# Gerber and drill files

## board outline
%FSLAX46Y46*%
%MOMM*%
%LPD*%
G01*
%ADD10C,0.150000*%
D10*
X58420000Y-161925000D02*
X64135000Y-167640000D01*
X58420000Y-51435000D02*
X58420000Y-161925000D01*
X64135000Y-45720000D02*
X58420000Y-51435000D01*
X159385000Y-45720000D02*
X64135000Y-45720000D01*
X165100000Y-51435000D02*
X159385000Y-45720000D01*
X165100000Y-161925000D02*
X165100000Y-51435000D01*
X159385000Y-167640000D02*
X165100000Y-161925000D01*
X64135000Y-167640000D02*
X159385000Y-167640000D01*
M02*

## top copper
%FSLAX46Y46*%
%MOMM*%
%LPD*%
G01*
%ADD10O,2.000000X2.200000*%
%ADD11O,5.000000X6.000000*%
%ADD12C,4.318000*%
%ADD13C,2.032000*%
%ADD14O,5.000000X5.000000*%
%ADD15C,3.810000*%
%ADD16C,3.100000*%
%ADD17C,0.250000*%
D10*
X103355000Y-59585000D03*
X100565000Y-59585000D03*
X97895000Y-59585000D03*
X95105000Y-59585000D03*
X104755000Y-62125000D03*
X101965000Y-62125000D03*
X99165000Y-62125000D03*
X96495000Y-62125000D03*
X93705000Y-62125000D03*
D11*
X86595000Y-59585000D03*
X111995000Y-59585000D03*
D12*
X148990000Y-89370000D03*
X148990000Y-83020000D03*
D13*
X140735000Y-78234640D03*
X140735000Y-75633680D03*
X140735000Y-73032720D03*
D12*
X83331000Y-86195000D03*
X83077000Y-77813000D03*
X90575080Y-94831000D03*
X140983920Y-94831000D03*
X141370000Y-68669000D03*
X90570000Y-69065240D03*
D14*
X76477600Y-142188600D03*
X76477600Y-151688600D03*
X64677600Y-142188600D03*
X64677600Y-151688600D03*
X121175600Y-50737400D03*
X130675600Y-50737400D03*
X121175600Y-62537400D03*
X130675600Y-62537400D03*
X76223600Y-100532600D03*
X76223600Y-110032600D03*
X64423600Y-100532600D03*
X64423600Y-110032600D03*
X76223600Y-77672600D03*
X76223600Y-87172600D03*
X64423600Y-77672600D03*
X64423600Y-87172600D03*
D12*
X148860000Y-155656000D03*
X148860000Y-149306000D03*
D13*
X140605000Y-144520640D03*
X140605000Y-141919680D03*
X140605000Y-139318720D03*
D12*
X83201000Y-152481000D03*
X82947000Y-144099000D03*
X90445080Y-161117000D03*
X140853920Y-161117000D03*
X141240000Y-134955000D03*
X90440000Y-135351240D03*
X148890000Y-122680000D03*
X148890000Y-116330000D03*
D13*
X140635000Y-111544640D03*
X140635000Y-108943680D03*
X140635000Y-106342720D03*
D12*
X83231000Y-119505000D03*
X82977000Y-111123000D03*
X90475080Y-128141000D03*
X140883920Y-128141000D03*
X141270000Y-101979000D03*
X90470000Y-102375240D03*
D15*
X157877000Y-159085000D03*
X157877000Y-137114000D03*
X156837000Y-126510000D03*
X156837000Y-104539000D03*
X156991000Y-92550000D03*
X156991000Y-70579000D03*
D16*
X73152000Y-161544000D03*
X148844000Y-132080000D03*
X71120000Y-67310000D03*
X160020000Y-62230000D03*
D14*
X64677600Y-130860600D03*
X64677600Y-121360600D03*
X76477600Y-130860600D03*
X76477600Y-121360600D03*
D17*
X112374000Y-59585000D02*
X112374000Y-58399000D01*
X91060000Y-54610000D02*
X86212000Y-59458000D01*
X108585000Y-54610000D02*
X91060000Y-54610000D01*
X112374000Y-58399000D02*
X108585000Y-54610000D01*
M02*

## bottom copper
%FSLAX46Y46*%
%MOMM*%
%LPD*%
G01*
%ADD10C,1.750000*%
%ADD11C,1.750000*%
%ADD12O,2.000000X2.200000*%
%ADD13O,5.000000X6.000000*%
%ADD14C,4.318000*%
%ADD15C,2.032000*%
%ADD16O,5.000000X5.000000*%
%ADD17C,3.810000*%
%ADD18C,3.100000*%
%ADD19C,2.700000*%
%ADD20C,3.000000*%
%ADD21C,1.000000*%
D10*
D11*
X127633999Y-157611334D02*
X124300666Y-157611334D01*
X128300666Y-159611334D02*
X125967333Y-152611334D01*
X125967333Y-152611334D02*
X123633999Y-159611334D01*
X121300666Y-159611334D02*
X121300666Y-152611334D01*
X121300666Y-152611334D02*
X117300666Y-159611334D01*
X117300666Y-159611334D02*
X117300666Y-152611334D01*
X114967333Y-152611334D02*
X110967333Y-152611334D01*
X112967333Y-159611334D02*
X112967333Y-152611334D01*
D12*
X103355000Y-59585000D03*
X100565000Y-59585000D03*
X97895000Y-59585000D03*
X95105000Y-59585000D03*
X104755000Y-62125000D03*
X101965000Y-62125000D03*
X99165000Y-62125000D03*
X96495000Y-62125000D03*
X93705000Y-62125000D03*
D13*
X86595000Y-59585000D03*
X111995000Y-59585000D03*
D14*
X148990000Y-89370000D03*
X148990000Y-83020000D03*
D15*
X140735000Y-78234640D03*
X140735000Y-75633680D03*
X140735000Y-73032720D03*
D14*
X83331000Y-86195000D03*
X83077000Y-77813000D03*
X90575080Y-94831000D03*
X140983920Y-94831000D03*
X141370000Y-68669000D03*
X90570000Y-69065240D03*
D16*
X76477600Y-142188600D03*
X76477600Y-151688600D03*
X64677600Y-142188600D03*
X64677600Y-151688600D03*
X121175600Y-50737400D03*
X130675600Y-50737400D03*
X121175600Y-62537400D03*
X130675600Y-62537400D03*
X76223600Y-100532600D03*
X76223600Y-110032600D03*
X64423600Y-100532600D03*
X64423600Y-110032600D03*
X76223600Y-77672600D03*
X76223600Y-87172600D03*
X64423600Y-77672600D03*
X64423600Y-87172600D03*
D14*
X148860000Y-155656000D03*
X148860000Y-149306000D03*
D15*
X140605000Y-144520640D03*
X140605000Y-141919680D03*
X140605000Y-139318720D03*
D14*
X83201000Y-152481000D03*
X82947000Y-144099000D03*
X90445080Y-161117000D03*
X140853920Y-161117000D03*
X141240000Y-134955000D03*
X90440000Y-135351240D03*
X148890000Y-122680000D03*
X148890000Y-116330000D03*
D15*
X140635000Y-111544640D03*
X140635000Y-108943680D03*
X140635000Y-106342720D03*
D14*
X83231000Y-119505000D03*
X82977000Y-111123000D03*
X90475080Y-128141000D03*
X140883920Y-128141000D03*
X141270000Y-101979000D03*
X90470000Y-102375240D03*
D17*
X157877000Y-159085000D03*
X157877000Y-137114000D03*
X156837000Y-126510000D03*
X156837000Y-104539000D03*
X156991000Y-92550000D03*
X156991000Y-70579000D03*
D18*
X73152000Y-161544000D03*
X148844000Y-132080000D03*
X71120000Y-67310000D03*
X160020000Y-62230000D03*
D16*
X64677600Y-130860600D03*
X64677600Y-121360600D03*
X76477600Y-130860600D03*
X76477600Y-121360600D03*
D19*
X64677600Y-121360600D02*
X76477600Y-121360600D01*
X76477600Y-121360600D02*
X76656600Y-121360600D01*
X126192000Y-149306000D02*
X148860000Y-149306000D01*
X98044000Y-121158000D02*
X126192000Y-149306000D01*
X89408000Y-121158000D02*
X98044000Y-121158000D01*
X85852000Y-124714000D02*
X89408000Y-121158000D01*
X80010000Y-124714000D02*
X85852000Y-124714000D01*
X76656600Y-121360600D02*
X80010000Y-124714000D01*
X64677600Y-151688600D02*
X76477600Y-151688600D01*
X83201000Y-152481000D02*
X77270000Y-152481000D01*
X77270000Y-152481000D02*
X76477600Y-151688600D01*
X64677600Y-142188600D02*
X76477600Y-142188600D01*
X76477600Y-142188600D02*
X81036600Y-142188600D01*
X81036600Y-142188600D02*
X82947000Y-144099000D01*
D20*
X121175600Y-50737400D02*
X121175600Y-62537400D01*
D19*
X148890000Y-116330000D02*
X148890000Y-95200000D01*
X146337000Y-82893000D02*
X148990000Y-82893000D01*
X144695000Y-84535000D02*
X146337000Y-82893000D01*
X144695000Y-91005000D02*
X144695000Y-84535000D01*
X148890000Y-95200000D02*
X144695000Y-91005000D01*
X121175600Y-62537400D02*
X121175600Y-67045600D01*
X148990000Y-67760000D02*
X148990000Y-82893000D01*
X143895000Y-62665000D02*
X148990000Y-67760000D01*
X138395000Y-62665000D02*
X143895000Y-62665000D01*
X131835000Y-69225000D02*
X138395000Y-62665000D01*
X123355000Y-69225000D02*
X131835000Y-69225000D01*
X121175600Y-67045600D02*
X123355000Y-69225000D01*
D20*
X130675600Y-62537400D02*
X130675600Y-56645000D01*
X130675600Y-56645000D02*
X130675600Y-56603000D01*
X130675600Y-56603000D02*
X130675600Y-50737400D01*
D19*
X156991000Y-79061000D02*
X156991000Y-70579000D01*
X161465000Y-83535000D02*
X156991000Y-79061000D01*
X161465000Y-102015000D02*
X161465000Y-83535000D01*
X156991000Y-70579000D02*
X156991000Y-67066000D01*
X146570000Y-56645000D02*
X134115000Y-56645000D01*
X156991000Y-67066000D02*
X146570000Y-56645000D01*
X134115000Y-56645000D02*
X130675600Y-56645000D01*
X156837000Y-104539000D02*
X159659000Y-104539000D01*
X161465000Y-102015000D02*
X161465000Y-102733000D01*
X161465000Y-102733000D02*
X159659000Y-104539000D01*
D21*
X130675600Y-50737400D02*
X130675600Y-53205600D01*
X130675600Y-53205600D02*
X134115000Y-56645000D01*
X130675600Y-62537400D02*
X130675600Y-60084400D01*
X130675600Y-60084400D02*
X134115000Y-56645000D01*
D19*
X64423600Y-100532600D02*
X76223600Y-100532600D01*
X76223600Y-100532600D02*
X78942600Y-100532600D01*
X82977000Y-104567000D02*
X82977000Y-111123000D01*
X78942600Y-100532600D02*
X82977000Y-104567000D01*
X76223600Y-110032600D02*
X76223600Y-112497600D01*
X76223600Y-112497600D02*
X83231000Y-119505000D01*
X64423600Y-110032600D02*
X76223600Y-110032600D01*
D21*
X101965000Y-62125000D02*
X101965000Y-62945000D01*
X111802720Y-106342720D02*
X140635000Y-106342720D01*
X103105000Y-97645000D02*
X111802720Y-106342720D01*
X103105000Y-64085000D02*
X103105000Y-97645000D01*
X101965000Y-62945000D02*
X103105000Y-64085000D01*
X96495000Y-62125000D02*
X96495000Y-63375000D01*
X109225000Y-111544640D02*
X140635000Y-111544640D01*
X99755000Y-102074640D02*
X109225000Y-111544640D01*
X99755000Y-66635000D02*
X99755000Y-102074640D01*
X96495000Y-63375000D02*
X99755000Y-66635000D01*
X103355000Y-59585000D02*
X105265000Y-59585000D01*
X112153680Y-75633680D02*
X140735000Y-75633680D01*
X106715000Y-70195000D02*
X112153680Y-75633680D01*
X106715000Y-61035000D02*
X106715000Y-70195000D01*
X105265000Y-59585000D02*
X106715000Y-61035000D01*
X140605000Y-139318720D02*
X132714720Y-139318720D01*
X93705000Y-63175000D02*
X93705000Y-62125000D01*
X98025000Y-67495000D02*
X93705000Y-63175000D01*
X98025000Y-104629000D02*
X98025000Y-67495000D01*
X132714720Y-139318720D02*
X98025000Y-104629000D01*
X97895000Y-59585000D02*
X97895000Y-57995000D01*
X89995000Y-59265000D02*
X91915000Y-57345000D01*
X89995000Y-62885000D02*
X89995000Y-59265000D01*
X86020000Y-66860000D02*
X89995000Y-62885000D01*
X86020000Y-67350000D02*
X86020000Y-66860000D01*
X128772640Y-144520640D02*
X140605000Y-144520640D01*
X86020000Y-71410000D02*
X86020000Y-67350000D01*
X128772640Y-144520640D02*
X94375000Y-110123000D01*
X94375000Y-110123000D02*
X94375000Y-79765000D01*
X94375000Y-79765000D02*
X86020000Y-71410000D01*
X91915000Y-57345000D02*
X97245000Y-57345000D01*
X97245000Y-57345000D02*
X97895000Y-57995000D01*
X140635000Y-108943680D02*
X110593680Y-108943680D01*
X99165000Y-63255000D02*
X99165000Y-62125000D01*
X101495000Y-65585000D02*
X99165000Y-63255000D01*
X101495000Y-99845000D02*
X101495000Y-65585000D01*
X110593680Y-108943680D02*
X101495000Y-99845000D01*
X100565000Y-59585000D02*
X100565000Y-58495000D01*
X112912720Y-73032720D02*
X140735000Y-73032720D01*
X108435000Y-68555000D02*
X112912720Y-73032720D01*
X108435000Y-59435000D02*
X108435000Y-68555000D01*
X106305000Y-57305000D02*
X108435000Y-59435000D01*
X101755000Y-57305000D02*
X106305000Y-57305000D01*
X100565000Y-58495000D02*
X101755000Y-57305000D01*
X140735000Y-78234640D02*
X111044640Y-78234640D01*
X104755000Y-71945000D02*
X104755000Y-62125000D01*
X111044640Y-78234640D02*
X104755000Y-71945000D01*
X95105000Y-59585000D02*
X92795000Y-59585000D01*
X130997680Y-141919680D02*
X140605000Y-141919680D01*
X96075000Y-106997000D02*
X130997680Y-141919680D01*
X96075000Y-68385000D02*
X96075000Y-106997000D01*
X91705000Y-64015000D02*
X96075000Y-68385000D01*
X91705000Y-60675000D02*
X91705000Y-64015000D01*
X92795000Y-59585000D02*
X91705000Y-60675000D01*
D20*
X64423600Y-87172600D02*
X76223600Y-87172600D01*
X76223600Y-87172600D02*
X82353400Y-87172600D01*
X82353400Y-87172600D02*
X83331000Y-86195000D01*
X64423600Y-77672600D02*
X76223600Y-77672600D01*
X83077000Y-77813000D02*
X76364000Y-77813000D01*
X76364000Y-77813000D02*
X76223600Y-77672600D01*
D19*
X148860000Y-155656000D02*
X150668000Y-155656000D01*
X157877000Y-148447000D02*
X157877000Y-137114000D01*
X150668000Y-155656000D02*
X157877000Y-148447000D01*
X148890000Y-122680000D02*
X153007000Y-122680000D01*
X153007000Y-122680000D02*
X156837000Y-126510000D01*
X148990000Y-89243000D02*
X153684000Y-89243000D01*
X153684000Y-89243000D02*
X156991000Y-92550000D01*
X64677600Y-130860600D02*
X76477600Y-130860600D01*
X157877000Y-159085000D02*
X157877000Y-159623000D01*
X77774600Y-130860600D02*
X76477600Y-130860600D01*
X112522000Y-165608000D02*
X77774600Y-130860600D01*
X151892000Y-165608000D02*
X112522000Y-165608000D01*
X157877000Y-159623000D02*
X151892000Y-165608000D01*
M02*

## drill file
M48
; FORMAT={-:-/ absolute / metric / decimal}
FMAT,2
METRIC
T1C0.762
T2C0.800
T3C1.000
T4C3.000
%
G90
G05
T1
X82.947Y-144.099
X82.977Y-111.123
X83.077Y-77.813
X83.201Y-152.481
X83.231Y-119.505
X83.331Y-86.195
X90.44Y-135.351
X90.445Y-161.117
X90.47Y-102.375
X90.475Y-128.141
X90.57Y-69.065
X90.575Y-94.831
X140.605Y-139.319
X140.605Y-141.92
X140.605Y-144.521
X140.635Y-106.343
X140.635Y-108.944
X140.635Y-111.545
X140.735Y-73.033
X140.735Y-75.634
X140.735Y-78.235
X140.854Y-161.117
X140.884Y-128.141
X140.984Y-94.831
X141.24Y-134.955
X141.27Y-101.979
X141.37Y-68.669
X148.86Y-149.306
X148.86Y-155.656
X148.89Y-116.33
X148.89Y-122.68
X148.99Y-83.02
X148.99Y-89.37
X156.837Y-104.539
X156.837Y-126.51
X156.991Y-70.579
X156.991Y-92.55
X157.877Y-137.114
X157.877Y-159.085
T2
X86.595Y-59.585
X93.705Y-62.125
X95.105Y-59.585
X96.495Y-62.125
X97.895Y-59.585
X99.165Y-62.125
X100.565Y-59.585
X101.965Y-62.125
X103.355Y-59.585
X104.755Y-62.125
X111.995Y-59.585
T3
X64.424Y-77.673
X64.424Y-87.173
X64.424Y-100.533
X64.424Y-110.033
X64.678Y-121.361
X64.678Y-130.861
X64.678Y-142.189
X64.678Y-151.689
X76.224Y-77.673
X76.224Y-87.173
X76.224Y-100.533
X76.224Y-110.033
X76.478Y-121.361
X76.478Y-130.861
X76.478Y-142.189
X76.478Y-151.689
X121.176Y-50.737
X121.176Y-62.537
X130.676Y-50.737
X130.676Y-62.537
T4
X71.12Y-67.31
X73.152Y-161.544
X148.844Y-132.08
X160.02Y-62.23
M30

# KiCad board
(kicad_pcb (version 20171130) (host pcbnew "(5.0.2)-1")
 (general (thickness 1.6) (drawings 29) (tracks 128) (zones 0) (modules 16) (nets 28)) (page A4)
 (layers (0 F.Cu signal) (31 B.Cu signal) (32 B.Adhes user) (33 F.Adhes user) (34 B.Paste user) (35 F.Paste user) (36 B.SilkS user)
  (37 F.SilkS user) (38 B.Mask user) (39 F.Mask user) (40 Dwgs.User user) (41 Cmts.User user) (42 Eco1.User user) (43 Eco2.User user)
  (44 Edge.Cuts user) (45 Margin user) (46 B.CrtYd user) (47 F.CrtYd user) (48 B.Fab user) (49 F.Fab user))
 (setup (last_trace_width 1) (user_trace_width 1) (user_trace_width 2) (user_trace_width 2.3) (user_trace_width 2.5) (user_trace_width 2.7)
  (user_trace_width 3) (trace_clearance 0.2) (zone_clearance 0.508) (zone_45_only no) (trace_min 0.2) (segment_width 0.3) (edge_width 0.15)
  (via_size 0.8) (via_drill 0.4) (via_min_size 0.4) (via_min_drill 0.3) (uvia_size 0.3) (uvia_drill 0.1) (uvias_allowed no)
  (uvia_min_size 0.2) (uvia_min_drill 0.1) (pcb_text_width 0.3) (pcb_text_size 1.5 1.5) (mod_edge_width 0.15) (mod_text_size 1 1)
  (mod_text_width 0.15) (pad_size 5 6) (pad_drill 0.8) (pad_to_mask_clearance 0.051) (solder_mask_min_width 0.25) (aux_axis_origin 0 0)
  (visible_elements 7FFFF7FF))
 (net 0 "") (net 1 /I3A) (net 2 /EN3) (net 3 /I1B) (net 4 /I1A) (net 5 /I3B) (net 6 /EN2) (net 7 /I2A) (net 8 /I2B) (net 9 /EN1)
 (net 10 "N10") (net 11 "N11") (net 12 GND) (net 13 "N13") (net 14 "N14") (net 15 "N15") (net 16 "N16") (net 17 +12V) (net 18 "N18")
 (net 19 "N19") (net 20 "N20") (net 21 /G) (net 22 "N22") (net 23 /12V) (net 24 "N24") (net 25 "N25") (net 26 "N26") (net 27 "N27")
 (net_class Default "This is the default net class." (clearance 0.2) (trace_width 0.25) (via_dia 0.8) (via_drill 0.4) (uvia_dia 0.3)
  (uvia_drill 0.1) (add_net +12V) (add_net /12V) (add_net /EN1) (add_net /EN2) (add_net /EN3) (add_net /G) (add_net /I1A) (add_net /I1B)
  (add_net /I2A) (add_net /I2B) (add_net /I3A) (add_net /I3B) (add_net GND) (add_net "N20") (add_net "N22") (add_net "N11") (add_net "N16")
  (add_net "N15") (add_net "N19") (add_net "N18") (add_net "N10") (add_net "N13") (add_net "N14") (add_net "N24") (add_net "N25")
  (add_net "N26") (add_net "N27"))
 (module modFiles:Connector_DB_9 (layer F.Cu) (at 93.705 62.125)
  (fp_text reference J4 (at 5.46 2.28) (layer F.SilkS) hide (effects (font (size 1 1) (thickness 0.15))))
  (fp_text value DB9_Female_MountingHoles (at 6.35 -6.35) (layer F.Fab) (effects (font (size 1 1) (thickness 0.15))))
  (pad 9 thru_hole oval (at 9.65 -2.54) (size 2 2.2) (drill 0.8) (layers *.Cu *.Mask) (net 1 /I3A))
  (pad 8 thru_hole oval (at 6.86 -2.54) (size 2 2.2) (drill 0.8) (layers *.Cu *.Mask) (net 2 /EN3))
  (pad 7 thru_hole oval (at 4.19 -2.54) (size 2 2.2) (drill 0.8) (layers *.Cu *.Mask) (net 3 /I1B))
  (pad 6 thru_hole oval (at 1.4 -2.54) (size 2 2.2) (drill 0.8) (layers *.Cu *.Mask) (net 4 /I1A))
  (pad 5 thru_hole oval (at 11.05 0) (size 2 2.2) (drill 0.8) (layers *.Cu *.Mask) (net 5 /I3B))
  (pad 4 thru_hole oval (at 8.26 0) (size 2 2.2) (drill 0.8) (layers *.Cu *.Mask) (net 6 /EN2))
  (pad 3 thru_hole oval (at 5.46 0) (size 2 2.2) (drill 0.8) (layers *.Cu *.Mask) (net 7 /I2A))
  (pad 2 thru_hole oval (at 2.79 0) (size 2 2.2) (drill 0.8) (layers *.Cu *.Mask) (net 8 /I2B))
  (pad 1 thru_hole oval (at 0 0) (size 2 2.2) (drill 0.8) (layers *.Cu *.Mask) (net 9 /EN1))
  (pad 0 thru_hole oval (at -7.11 -2.54) (size 5 6) (drill 0.8) (layers *.Cu *.Mask) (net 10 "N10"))
  (pad 0 thru_hole oval (at 18.29 -2.54) (size 5 6) (drill 0.8) (layers *.Cu *.Mask) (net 10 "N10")))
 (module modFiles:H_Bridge (layer F.Cu) (at 139.465 83.655)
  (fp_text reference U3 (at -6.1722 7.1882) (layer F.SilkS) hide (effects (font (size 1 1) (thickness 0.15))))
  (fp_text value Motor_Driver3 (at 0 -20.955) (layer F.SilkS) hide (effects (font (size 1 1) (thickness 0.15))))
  (pad 6 thru_hole circle (at 9.525 5.715) (size 4.318 4.318) (drill 0.762) (layers *.Cu *.Mask F.SilkS) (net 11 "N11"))
  (pad 7 thru_hole circle (at 9.525 -0.635) (size 4.318 4.318) (drill 0.762) (layers *.Cu *.Mask F.SilkS) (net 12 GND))
  (pad 5 thru_hole circle (at 1.27 -5.42036) (size 2.032 2.032) (drill 0.762) (layers *.Cu *.Mask F.SilkS) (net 5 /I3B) (clearance -0.254))
  (pad 4 thru_hole circle (at 1.27 -8.02132) (size 2.032 2.032) (drill 0.762) (layers *.Cu *.Mask F.SilkS) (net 1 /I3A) (clearance -0.254))
  (pad 3 thru_hole circle (at 1.27 -10.62228) (size 2.032 2.032) (drill 0.762) (layers *.Cu *.Mask F.SilkS) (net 2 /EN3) (clearance -0.254))
  (pad 1 thru_hole circle (at -56.134 2.54) (size 4.318 4.318) (drill 0.762) (layers *.Cu *.Mask F.SilkS) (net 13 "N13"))
  (pad 2 thru_hole circle (at -56.388 -5.842) (size 4.318 4.318) (drill 0.762) (layers *.Cu *.Mask F.SilkS) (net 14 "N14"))
  (pad "" thru_hole circle (at -48.88992 11.176) (size 4.318 4.318) (drill 0.762) (layers *.Cu *.Mask F.SilkS))
  (pad "" thru_hole circle (at 1.51892 11.176) (size 4.318 4.318) (drill 0.762) (layers *.Cu *.Mask F.SilkS))
  (pad "" thru_hole circle (at 1.905 -14.986) (size 4.318 4.318) (drill 0.762) (layers *.Cu *.Mask F.SilkS))
  (pad "" thru_hole circle (at -48.895 -14.58976) (size 4.318 4.318) (drill 0.762) (layers *.Cu *.Mask F.SilkS)))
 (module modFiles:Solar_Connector (layer F.Cu) (at 70.104 147.066 90)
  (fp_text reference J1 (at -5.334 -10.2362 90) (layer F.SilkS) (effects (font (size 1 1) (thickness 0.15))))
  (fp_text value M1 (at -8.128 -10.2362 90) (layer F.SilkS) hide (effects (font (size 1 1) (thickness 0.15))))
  (pad 2 thru_hole oval (at 4.8774 6.3736 180) (size 5 5) (drill 1) (layers *.Cu *.Mask F.SilkS) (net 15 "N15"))
  (pad 1 thru_hole oval (at -4.6226 6.3736 180) (size 5 5) (drill 1) (layers *.Cu *.Mask F.SilkS) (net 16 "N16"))
  (pad 2 thru_hole oval (at 4.8774 -5.4264 180) (size 5 5) (drill 1) (layers *.Cu *.Mask F.SilkS) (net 15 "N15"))
  (pad 1 thru_hole oval (at -4.6226 -5.4264 180) (size 5 5) (drill 1) (layers *.Cu *.Mask F.SilkS) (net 16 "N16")))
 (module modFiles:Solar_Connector (layer F.Cu) (at 126.053 57.111 180)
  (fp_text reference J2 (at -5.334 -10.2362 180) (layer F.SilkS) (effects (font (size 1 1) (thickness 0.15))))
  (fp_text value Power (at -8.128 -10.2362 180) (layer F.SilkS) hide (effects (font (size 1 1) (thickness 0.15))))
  (pad 2 thru_hole oval (at 4.8774 6.3736 270) (size 5 5) (drill 1) (layers *.Cu *.Mask F.SilkS) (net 12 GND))
  (pad 1 thru_hole oval (at -4.6226 6.3736 270) (size 5 5) (drill 1) (layers *.Cu *.Mask F.SilkS) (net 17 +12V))
  (pad 2 thru_hole oval (at 4.8774 -5.4264 270) (size 5 5) (drill 1) (layers *.Cu *.Mask F.SilkS) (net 12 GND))
  (pad 1 thru_hole oval (at -4.6226 -5.4264 270) (size 5 5) (drill 1) (layers *.Cu *.Mask F.SilkS) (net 17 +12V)))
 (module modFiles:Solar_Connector (layer F.Cu) (at 69.85 105.41 90)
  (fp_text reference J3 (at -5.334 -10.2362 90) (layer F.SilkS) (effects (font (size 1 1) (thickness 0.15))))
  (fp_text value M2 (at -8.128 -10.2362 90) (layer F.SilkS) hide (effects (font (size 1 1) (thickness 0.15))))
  (pad 2 thru_hole oval (at 4.8774 6.3736 180) (size 5 5) (drill 1) (layers *.Cu *.Mask F.SilkS) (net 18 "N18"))
  (pad 1 thru_hole oval (at -4.6226 6.3736 180) (size 5 5) (drill 1) (layers *.Cu *.Mask F.SilkS) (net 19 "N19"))
  (pad 2 thru_hole oval (at 4.8774 -5.4264 180) (size 5 5) (drill 1) (layers *.Cu *.Mask F.SilkS) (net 18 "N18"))
  (pad 1 thru_hole oval (at -4.6226 -5.4264 180) (size 5 5) (drill 1) (layers *.Cu *.Mask F.SilkS) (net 19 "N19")))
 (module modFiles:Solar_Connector (layer F.Cu) (at 69.85 82.55 90)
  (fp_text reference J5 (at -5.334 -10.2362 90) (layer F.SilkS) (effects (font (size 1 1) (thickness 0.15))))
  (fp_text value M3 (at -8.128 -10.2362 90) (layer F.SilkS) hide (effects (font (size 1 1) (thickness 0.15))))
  (pad 2 thru_hole oval (at 4.8774 6.3736 180) (size 5 5) (drill 1) (layers *.Cu *.Mask F.SilkS) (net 14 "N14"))
  (pad 1 thru_hole oval (at -4.6226 6.3736 180) (size 5 5) (drill 1) (layers *.Cu *.Mask F.SilkS) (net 13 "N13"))
  (pad 2 thru_hole oval (at 4.8774 -5.4264 180) (size 5 5) (drill 1) (layers *.Cu *.Mask F.SilkS) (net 14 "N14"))
  (pad 1 thru_hole oval (at -4.6226 -5.4264 180) (size 5 5) (drill 1) (layers *.Cu *.Mask F.SilkS) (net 13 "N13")))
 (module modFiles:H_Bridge (layer F.Cu) (at 139.335 149.941)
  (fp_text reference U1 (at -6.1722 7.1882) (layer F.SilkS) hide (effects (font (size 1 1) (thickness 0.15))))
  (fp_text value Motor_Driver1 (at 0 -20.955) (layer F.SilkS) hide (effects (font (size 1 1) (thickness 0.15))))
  (pad 6 thru_hole circle (at 9.525 5.715) (size 4.318 4.318) (drill 0.762) (layers *.Cu *.Mask F.SilkS) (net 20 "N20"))
  (pad 7 thru_hole circle (at 9.525 -0.635) (size 4.318 4.318) (drill 0.762) (layers *.Cu *.Mask F.SilkS) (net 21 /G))
  (pad 5 thru_hole circle (at 1.27 -5.42036) (size 2.032 2.032) (drill 0.762) (layers *.Cu *.Mask F.SilkS) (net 3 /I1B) (clearance -0.254))
  (pad 4 thru_hole circle (at 1.27 -8.02132) (size 2.032 2.032) (drill 0.762) (layers *.Cu *.Mask F.SilkS) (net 4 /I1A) (clearance -0.254))
  (pad 3 thru_hole circle (at 1.27 -10.62228) (size 2.032 2.032) (drill 0.762) (layers *.Cu *.Mask F.SilkS) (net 9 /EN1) (clearance -0.254))
  (pad 1 thru_hole circle (at -56.134 2.54) (size 4.318 4.318) (drill 0.762) (layers *.Cu *.Mask F.SilkS) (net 16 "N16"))
  (pad 2 thru_hole circle (at -56.388 -5.842) (size 4.318 4.318) (drill 0.762) (layers *.Cu *.Mask F.SilkS) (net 15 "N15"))
  (pad "" thru_hole circle (at -48.88992 11.176) (size 4.318 4.318) (drill 0.762) (layers *.Cu *.Mask F.SilkS))
  (pad "" thru_hole circle (at 1.51892 11.176) (size 4.318 4.318) (drill 0.762) (layers *.Cu *.Mask F.SilkS))
  (pad "" thru_hole circle (at 1.905 -14.986) (size 4.318 4.318) (drill 0.762) (layers *.Cu *.Mask F.SilkS))
  (pad "" thru_hole circle (at -48.895 -14.58976) (size 4.318 4.318) (drill 0.762) (layers *.Cu *.Mask F.SilkS)))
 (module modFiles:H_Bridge (layer F.Cu) (at 139.365 116.965)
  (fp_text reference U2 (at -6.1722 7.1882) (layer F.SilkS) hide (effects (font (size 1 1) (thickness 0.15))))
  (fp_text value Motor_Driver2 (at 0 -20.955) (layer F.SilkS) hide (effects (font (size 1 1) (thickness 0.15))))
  (pad 6 thru_hole circle (at 9.525 5.715) (size 4.318 4.318) (drill 0.762) (layers *.Cu *.Mask F.SilkS) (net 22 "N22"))
  (pad 7 thru_hole circle (at 9.525 -0.635) (size 4.318 4.318) (drill 0.762) (layers *.Cu *.Mask F.SilkS) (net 12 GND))
  (pad 5 thru_hole circle (at 1.27 -5.42036) (size 2.032 2.032) (drill 0.762) (layers *.Cu *.Mask F.SilkS) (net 8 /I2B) (clearance -0.254))
  (pad 4 thru_hole circle (at 1.27 -8.02132) (size 2.032 2.032) (drill 0.762) (layers *.Cu *.Mask F.SilkS) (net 7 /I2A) (clearance -0.254))
  (pad 3 thru_hole circle (at 1.27 -10.62228) (size 2.032 2.032) (drill 0.762) (layers *.Cu *.Mask F.SilkS) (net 6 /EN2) (clearance -0.254))
  (pad 1 thru_hole circle (at -56.134 2.54) (size 4.318 4.318) (drill 0.762) (layers *.Cu *.Mask F.SilkS) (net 19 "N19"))
  (pad 2 thru_hole circle (at -56.388 -5.842) (size 4.318 4.318) (drill 0.762) (layers *.Cu *.Mask F.SilkS) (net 18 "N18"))
  (pad "" thru_hole circle (at -48.88992 11.176) (size 4.318 4.318) (drill 0.762) (layers *.Cu *.Mask F.SilkS))
  (pad "" thru_hole circle (at 1.51892 11.176) (size 4.318 4.318) (drill 0.762) (layers *.Cu *.Mask F.SilkS))
  (pad "" thru_hole circle (at 1.905 -14.986) (size 4.318 4.318) (drill 0.762) (layers *.Cu *.Mask F.SilkS))
  (pad "" thru_hole circle (at -48.895 -14.58976) (size 4.318 4.318) (drill 0.762) (layers *.Cu *.Mask F.SilkS)))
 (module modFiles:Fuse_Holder (layer F.Cu) (at 157.369 147.909 270)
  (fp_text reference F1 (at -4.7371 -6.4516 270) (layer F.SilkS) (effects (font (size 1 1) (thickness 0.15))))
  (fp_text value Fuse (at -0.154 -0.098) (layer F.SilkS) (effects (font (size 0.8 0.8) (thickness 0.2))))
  (pad 1 thru_hole circle (at 11.176 -0.508) (size 3.81 3.81) (drill 0.762) (layers *.Cu *.Mask F.SilkS) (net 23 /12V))
  (pad 2 thru_hole circle (at -10.795 -0.508) (size 3.81 3.81) (drill 0.762) (layers *.Cu *.Mask F.SilkS) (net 20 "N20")))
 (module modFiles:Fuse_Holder (layer F.Cu) (at 157.345 115.715 90)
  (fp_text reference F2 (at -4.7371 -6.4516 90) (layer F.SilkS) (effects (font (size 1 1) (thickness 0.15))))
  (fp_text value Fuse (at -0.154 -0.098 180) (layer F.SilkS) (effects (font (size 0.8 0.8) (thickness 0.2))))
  (pad 2 thru_hole circle (at -10.795 -0.508 180) (size 3.81 3.81) (drill 0.762) (layers *.Cu *.Mask F.SilkS) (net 22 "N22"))
  (pad 1 thru_hole circle (at 11.176 -0.508 180) (size 3.81 3.81) (drill 0.762) (layers *.Cu *.Mask F.SilkS) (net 17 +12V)))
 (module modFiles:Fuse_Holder (layer F.Cu) (at 157.499 81.755 90)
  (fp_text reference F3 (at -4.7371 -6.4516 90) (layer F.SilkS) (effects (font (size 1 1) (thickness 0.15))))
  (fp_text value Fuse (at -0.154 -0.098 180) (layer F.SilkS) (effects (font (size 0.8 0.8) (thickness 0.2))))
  (pad 2 thru_hole circle (at -10.795 -0.508 180) (size 3.81 3.81) (drill 0.762) (layers *.Cu *.Mask F.SilkS) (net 11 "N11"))
  (pad 1 thru_hole circle (at 11.176 -0.508 180) (size 3.81 3.81) (drill 0.762) (layers *.Cu *.Mask F.SilkS) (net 17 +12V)))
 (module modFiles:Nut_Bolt (layer F.Cu) (at 73.152 161.544 90)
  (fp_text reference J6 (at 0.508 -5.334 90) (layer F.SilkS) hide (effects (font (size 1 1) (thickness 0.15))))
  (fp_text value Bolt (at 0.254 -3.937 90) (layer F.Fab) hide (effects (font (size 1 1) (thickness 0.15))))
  (pad 1 thru_hole circle (at 0 0 90) (size 3.1 3.1) (drill 3) (layers *.Cu *.Mask) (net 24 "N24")))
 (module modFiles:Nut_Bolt (layer F.Cu) (at 148.844 132.08 90)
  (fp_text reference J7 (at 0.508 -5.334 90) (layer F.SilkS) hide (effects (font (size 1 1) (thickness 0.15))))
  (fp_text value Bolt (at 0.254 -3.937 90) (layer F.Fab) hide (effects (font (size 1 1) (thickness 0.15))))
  (pad 1 thru_hole circle (at 0 0 90) (size 3.1 3.1) (drill 3) (layers *.Cu *.Mask) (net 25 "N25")))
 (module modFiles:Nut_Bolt (layer F.Cu) (at 71.12 67.31 90)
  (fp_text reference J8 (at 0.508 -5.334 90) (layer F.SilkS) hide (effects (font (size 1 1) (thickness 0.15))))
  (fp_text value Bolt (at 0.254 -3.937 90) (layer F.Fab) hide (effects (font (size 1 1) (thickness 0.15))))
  (pad 1 thru_hole circle (at 0 0 90) (size 3.1 3.1) (drill 3) (layers *.Cu *.Mask) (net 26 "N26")))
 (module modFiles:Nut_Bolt (layer F.Cu) (at 160.02 62.23 90)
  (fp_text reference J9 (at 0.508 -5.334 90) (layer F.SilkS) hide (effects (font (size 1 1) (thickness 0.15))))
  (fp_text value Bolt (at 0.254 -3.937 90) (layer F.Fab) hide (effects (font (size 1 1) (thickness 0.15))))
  (pad 1 thru_hole circle (at 0 0 90) (size 3.1 3.1) (drill 3) (layers *.Cu *.Mask) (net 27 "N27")))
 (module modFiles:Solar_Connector (layer F.Cu) (at 70.104 126.238 90)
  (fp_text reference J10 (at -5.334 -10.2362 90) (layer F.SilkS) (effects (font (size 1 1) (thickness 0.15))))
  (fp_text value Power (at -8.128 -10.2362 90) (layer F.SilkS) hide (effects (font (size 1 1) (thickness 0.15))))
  (pad 1 thru_hole oval (at -4.6226 -5.4264 180) (size 5 5) (drill 1) (layers *.Cu *.Mask F.SilkS) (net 23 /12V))
  (pad 2 thru_hole oval (at 4.8774 -5.4264 180) (size 5 5) (drill 1) (layers *.Cu *.Mask F.SilkS) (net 21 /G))
  (pad 1 thru_hole oval (at -4.6226 6.3736 180) (size 5 5) (drill 1) (layers *.Cu *.Mask F.SilkS) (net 23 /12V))
  (pad 2 thru_hole oval (at 4.8774 6.3736 180) (size 5 5) (drill 1) (layers *.Cu *.Mask F.SilkS) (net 21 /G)))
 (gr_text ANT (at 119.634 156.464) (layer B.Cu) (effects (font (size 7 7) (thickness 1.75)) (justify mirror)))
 (gr_line (start 58.42 161.925) (end 64.135 167.64) (angle 90) (layer Edge.Cuts) (width 0.15))
 (gr_line (start 58.42 51.435) (end 58.42 161.925) (angle 90) (layer Edge.Cuts) (width 0.15))
 (gr_line (start 64.135 45.72) (end 58.42 51.435) (angle 90) (layer Edge.Cuts) (width 0.15))
 (gr_line (start 159.385 45.72) (end 64.135 45.72) (angle 90) (layer Edge.Cuts) (width 0.15))
 (gr_line (start 165.1 51.435) (end 159.385 45.72) (angle 90) (layer Edge.Cuts) (width 0.15))
 (gr_line (start 165.1 161.925) (end 165.1 51.435) (angle 90) (layer Edge.Cuts) (width 0.15))
 (gr_line (start 159.385 167.64) (end 165.1 161.925) (angle 90) (layer Edge.Cuts) (width 0.15))
 (gr_line (start 64.135 167.64) (end 159.385 167.64) (angle 90) (layer Edge.Cuts) (width 0.15))
 (segment (start 64.6776 121.3606) (end 76.4776 121.3606) (width 2.7) (layer B.Cu) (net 21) (status C00030))
 (segment (start 76.4776 121.3606) (end 76.6566 121.3606) (width 2.7) (layer B.Cu) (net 21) (status C00030))
 (segment (start 126.192 149.306) (end 148.86 149.306) (width 2.7) (layer B.Cu) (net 21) (status 800020))
 (segment (start 98.044 121.158) (end 126.192 149.306) (width 2.7) (layer B.Cu) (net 21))
 (segment (start 89.408 121.158) (end 98.044 121.158) (width 2.7) (layer B.Cu) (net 21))
 (segment (start 85.852 124.714) (end 89.408 121.158) (width 2.7) (layer B.Cu) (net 21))
 (segment (start 80.01 124.714) (end 85.852 124.714) (width 2.7) (layer B.Cu) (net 21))
 (segment (start 76.6566 121.3606) (end 80.01 124.714) (width 2.7) (layer B.Cu) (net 21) (status 400010))
 (segment (start 64.6776 151.6886) (end 76.4776 151.6886) (width 2.7) (layer B.Cu) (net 16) (status C00030))
 (segment (start 83.201 152.481) (end 77.27 152.481) (width 2.7) (layer B.Cu) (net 16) (status C00030))
 (segment (start 77.27 152.481) (end 76.4776 151.6886) (width 2.7) (layer B.Cu) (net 16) (status C00030))
 (segment (start 64.6776 142.1886) (end 76.4776 142.1886) (width 2.7) (layer B.Cu) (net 15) (status C00030))
 (segment (start 76.4776 142.1886) (end 81.0366 142.1886) (width 2.7) (layer B.Cu) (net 15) (status 400010))
 (segment (start 81.0366 142.1886) (end 82.947 144.099) (width 2.7) (layer B.Cu) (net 15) (status 800020))
 (segment (start 121.1756 50.7374) (end 121.1756 62.5374) (width 3) (layer B.Cu) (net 12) (status C00030))
 (segment (start 148.89 116.33) (end 148.89 95.2) (width 2.7) (layer B.Cu) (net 12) (status 400010))
 (segment (start 146.337 82.893) (end 148.99 82.893) (width 2.7) (layer B.Cu) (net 12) (status 800020))
 (segment (start 144.695 84.535) (end 146.337 82.893) (width 2.7) (layer B.Cu) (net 12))
 (segment (start 144.695 91.005) (end 144.695 84.535) (width 2.7) (layer B.Cu) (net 12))
 (segment (start 148.89 95.2) (end 144.695 91.005) (width 2.7) (layer B.Cu) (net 12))
 (segment (start 121.1756 62.5374) (end 121.1756 67.0456) (width 2.7) (layer B.Cu) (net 12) (status 400010))
 (segment (start 148.99 67.76) (end 148.99 82.893) (width 2.7) (layer B.Cu) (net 12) (status 800020))
 (segment (start 143.895 62.665) (end 148.99 67.76) (width 2.7) (layer B.Cu) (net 12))
 (segment (start 138.395 62.665) (end 143.895 62.665) (width 2.7) (layer B.Cu) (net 12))
 (segment (start 131.835 69.225) (end 138.395 62.665) (width 2.7) (layer B.Cu) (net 12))
 (segment (start 123.355 69.225) (end 131.835 69.225) (width 2.7) (layer B.Cu) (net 12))
 (segment (start 121.1756 67.0456) (end 123.355 69.225) (width 2.7) (layer B.Cu) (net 12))
 (segment (start 130.6756 62.5374) (end 130.6756 56.645) (width 3) (layer B.Cu) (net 17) (status 400010))
 (segment (start 130.6756 56.645) (end 130.6756 56.603) (width 3) (layer B.Cu) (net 17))
 (segment (start 130.6756 56.603) (end 130.6756 50.7374) (width 3) (layer B.Cu) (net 17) (status 800020))
 (segment (start 156.991 79.061) (end 156.991 70.579) (width 2.7) (layer B.Cu) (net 17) (status 800020))
 (segment (start 161.465 83.535) (end 156.991 79.061) (width 2.7) (layer B.Cu) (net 17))
 (segment (start 161.465 102.015) (end 161.465 83.535) (width 2.7) (layer B.Cu) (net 17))
 (segment (start 156.991 70.579) (end 156.991 67.066) (width 2.7) (layer B.Cu) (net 17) (status 400010))
 (segment (start 146.57 56.645) (end 134.115 56.645) (width 2.7) (layer B.Cu) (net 17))
 (segment (start 156.991 67.066) (end 146.57 56.645) (width 2.7) (layer B.Cu) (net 17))
 (segment (start 134.115 56.645) (end 130.6756 56.645) (width 2.7) (layer B.Cu) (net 17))
 (segment (start 156.837 104.539) (end 159.659 104.539) (width 2.7) (layer B.Cu) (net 17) (status 400010))
 (segment (start 161.465 102.015) (end 161.465 102.733) (width 2.7) (layer B.Cu) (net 17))
 (segment (start 161.465 102.733) (end 159.659 104.539) (width 2.7) (layer B.Cu) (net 17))
 (segment (start 130.6756 50.7374) (end 130.6756 53.2056) (width 1) (layer B.Cu) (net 17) (status C00000))
 (segment (start 130.6756 53.2056) (end 134.115 56.645) (width 1) (layer B.Cu) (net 17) (status 400000))
 (segment (start 130.6756 62.5374) (end 130.6756 60.0844) (width 1) (layer B.Cu) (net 17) (status C00000))
 (segment (start 130.6756 60.0844) (end 134.115 56.645) (width 1) (layer B.Cu) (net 17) (status 400000))
 (segment (start 64.4236 100.5326) (end 76.2236 100.5326) (width 2.7) (layer B.Cu) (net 18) (status C00030))
 (segment (start 76.2236 100.5326) (end 78.9426 100.5326) (width 2.7) (layer B.Cu) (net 18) (status 400010))
 (segment (start 82.977 104.567) (end 82.977 111.123) (width 2.7) (layer B.Cu) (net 18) (status 800020))
 (segment (start 78.9426 100.5326) (end 82.977 104.567) (width 2.7) (layer B.Cu) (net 18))
 (segment (start 76.2236 110.0326) (end 76.2236 112.4976) (width 2.7) (layer B.Cu) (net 19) (status C00030))
 (segment (start 76.2236 112.4976) (end 83.231 119.505) (width 2.7) (layer B.Cu) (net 19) (status C00030))
 (segment (start 64.4236 110.0326) (end 76.2236 110.0326) (width 2.7) (layer B.Cu) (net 19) (status C00030))
 (segment (start 101.965 62.125) (end 101.965 62.945) (width 1) (layer B.Cu) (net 6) (status 400030))
 (segment (start 111.80272 106.34272) (end 140.635 106.34272) (width 1) (layer B.Cu) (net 6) (status 800020))
 (segment (start 103.105 97.645) (end 111.80272 106.34272) (width 1) (layer B.Cu) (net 6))
 (segment (start 103.105 64.085) (end 103.105 97.645) (width 1) (layer B.Cu) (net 6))
 (segment (start 101.965 62.945) (end 103.105 64.085) (width 1) (layer B.Cu) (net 6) (status 10))
 (segment (start 96.495 62.125) (end 96.495 63.375) (width 1) (layer B.Cu) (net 8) (status 400010))
 (segment (start 109.225 111.54464) (end 140.635 111.54464) (width 1) (layer B.Cu) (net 8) (status 800020))
 (segment (start 99.755 102.07464) (end 109.225 111.54464) (width 1) (layer B.Cu) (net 8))
 (segment (start 99.755 66.635) (end 99.755 102.07464) (width 1) (layer B.Cu) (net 8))
 (segment (start 96.495 63.375) (end 99.755 66.635) (width 1) (layer B.Cu) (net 8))
 (segment (start 103.355 59.585) (end 105.265 59.585) (width 1) (layer B.Cu) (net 1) (status 400010))
 (segment (start 112.15368 75.63368) (end 140.735 75.63368) (width 1) (layer B.Cu) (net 1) (status 800020))
 (segment (start 106.715 70.195) (end 112.15368 75.63368) (width 1) (layer B.Cu) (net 1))
 (segment (start 106.715 61.035) (end 106.715 70.195) (width 1) (layer B.Cu) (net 1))
 (segment (start 105.265 59.585) (end 106.715 61.035) (width 1) (layer B.Cu) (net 1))
 (segment (start 140.605 139.31872) (end 132.71472 139.31872) (width 1) (layer B.Cu) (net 9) (status 400010))
 (segment (start 93.705 63.175) (end 93.705 62.125) (width 1) (layer B.Cu) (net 9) (status 800030))
 (segment (start 98.025 67.495) (end 93.705 63.175) (width 1) (layer B.Cu) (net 9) (status 20))
 (segment (start 98.025 104.629) (end 98.025 67.495) (width 1) (layer B.Cu) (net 9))
 (segment (start 132.71472 139.31872) (end 98.025 104.629) (width 1) (layer B.Cu) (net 9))
 (segment (start 97.895 59.585) (end 97.895 57.995) (width 1) (layer B.Cu) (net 3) (status 400010))
 (segment (start 89.995 59.265) (end 91.915 57.345) (width 1) (layer B.Cu) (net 3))
 (segment (start 89.995 62.885) (end 89.995 59.265) (width 1) (layer B.Cu) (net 3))
 (segment (start 86.02 66.86) (end 89.995 62.885) (width 1) (layer B.Cu) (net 3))
 (segment (start 86.02 67.35) (end 86.02 66.86) (width 1) (layer B.Cu) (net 3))
 (segment (start 128.77264 144.52064) (end 140.605 144.52064) (width 1) (layer B.Cu) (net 3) (status 800020))
 (segment (start 86.02 71.41) (end 86.02 67.35) (width 1) (layer B.Cu) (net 3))
 (segment (start 128.77264 144.52064) (end 94.375 110.123) (width 1) (layer B.Cu) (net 3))
 (segment (start 94.375 110.123) (end 94.375 79.765) (width 1) (layer B.Cu) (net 3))
 (segment (start 94.375 79.765) (end 86.02 71.41) (width 1) (layer B.Cu) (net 3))
 (segment (start 91.915 57.345) (end 97.245 57.345) (width 1) (layer B.Cu) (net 3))
 (segment (start 97.245 57.345) (end 97.895 57.995) (width 1) (layer B.Cu) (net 3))
 (segment (start 140.635 108.94368) (end 110.59368 108.94368) (width 1) (layer B.Cu) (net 7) (status 400010))
 (segment (start 99.165 63.255) (end 99.165 62.125) (width 1) (layer B.Cu) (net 7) (status 800020))
 (segment (start 101.495 65.585) (end 99.165 63.255) (width 1) (layer B.Cu) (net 7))
 (segment (start 101.495 99.845) (end 101.495 65.585) (width 1) (layer B.Cu) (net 7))
 (segment (start 110.59368 108.94368) (end 101.495 99.845) (width 1) (layer B.Cu) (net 7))
 (segment (start 100.565 59.585) (end 100.565 58.495) (width 1) (layer B.Cu) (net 2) (status 400030))
 (segment (start 112.91272 73.03272) (end 140.735 73.03272) (width 1) (layer B.Cu) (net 2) (status 800020))
 (segment (start 108.435 68.555) (end 112.91272 73.03272) (width 1) (layer B.Cu) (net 2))
 (segment (start 108.435 59.435) (end 108.435 68.555) (width 1) (layer B.Cu) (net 2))
 (segment (start 106.305 57.305) (end 108.435 59.435) (width 1) (layer B.Cu) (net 2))
 (segment (start 101.755 57.305) (end 106.305 57.305) (width 1) (layer B.Cu) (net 2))
 (segment (start 100.565 58.495) (end 101.755 57.305) (width 1) (layer B.Cu) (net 2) (status 10))
 (segment (start 140.735 78.23464) (end 111.04464 78.23464) (width 1) (layer B.Cu) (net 5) (status 400010))
 (segment (start 104.755 71.945) (end 104.755 62.125) (width 1) (layer B.Cu) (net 5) (status 800020))
 (segment (start 111.04464 78.23464) (end 104.755 71.945) (width 1) (layer B.Cu) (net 5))
 (segment (start 95.105 59.585) (end 92.795 59.585) (width 1) (layer B.Cu) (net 4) (status 400010))
 (segment (start 130.99768 141.91968) (end 140.605 141.91968) (width 1) (layer B.Cu) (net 4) (status 800020))
 (segment (start 96.075 106.997) (end 130.99768 141.91968) (width 1) (layer B.Cu) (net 4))
 (segment (start 96.075 68.385) (end 96.075 106.997) (width 1) (layer B.Cu) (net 4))
 (segment (start 91.705 64.015) (end 96.075 68.385) (width 1) (layer B.Cu) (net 4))
 (segment (start 91.705 60.675) (end 91.705 64.015) (width 1) (layer B.Cu) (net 4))
 (segment (start 92.795 59.585) (end 91.705 60.675) (width 1) (layer B.Cu) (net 4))
 (segment (start 64.4236 87.1726) (end 76.2236 87.1726) (width 3) (layer B.Cu) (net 13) (status C00030))
 (segment (start 76.2236 87.1726) (end 82.3534 87.1726) (width 3) (layer B.Cu) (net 13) (status C00030))
 (segment (start 82.3534 87.1726) (end 83.331 86.195) (width 3) (layer B.Cu) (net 13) (status C00030))
 (segment (start 64.4236 77.6726) (end 76.2236 77.6726) (width 3) (layer B.Cu) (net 14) (status C00030))
 (segment (start 83.077 77.813) (end 76.364 77.813) (width 3) (layer B.Cu) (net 14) (status C00030))
 (segment (start 76.364 77.813) (end 76.2236 77.6726) (width 3) (layer B.Cu) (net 14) (status C00030))
 (segment (start 148.86 155.656) (end 150.668 155.656) (width 2.7) (layer B.Cu) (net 20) (status C00030))
 (segment (start 157.877 148.447) (end 157.877 137.114) (width 2.7) (layer B.Cu) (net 20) (status 800020))
 (segment (start 150.668 155.656) (end 157.877 148.447) (width 2.7) (layer B.Cu) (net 20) (status 400010))
 (segment (start 148.89 122.68) (end 153.007 122.68) (width 2.7) (layer B.Cu) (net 22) (status 400010))
 (segment (start 153.007 122.68) (end 156.837 126.51) (width 2.7) (layer B.Cu) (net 22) (status 800020))
 (segment (start 148.99 89.243) (end 153.684 89.243) (width 2.7) (layer B.Cu) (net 11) (status 400010))
 (segment (start 153.684 89.243) (end 156.991 92.55) (width 2.7) (layer B.Cu) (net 11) (status 800020))
 (segment (start 64.6776 130.8606) (end 76.4776 130.8606) (width 2.7) (layer B.Cu) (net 23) (status C00030))
 (segment (start 157.877 159.085) (end 157.877 159.623) (width 2.7) (layer B.Cu) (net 23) (status C00030))
 (segment (start 77.7746 130.8606) (end 76.4776 130.8606) (width 2.7) (layer B.Cu) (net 23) (status C00030))
 (segment (start 112.522 165.608) (end 77.7746 130.8606) (width 2.7) (layer B.Cu) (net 23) (status 800020))
 (segment (start 151.892 165.608) (end 112.522 165.608) (width 2.7) (layer B.Cu) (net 23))
 (segment (start 157.877 159.623) (end 151.892 165.608) (width 2.7) (layer B.Cu) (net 23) (status 400010))
 (segment (start 112.374 59.585) (end 112.374 58.399) (width 0.25) (layer F.Cu) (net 10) (status C00030))
 (segment (start 91.06 54.61) (end 86.212 59.458) (width 0.25) (layer F.Cu) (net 10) (status 800020))
 (segment (start 108.585 54.61) (end 91.06 54.61) (width 0.25) (layer F.Cu) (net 10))
 (segment (start 112.374 58.399) (end 108.585 54.61) (width 0.25) (layer F.Cu) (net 10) (status 400010)))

